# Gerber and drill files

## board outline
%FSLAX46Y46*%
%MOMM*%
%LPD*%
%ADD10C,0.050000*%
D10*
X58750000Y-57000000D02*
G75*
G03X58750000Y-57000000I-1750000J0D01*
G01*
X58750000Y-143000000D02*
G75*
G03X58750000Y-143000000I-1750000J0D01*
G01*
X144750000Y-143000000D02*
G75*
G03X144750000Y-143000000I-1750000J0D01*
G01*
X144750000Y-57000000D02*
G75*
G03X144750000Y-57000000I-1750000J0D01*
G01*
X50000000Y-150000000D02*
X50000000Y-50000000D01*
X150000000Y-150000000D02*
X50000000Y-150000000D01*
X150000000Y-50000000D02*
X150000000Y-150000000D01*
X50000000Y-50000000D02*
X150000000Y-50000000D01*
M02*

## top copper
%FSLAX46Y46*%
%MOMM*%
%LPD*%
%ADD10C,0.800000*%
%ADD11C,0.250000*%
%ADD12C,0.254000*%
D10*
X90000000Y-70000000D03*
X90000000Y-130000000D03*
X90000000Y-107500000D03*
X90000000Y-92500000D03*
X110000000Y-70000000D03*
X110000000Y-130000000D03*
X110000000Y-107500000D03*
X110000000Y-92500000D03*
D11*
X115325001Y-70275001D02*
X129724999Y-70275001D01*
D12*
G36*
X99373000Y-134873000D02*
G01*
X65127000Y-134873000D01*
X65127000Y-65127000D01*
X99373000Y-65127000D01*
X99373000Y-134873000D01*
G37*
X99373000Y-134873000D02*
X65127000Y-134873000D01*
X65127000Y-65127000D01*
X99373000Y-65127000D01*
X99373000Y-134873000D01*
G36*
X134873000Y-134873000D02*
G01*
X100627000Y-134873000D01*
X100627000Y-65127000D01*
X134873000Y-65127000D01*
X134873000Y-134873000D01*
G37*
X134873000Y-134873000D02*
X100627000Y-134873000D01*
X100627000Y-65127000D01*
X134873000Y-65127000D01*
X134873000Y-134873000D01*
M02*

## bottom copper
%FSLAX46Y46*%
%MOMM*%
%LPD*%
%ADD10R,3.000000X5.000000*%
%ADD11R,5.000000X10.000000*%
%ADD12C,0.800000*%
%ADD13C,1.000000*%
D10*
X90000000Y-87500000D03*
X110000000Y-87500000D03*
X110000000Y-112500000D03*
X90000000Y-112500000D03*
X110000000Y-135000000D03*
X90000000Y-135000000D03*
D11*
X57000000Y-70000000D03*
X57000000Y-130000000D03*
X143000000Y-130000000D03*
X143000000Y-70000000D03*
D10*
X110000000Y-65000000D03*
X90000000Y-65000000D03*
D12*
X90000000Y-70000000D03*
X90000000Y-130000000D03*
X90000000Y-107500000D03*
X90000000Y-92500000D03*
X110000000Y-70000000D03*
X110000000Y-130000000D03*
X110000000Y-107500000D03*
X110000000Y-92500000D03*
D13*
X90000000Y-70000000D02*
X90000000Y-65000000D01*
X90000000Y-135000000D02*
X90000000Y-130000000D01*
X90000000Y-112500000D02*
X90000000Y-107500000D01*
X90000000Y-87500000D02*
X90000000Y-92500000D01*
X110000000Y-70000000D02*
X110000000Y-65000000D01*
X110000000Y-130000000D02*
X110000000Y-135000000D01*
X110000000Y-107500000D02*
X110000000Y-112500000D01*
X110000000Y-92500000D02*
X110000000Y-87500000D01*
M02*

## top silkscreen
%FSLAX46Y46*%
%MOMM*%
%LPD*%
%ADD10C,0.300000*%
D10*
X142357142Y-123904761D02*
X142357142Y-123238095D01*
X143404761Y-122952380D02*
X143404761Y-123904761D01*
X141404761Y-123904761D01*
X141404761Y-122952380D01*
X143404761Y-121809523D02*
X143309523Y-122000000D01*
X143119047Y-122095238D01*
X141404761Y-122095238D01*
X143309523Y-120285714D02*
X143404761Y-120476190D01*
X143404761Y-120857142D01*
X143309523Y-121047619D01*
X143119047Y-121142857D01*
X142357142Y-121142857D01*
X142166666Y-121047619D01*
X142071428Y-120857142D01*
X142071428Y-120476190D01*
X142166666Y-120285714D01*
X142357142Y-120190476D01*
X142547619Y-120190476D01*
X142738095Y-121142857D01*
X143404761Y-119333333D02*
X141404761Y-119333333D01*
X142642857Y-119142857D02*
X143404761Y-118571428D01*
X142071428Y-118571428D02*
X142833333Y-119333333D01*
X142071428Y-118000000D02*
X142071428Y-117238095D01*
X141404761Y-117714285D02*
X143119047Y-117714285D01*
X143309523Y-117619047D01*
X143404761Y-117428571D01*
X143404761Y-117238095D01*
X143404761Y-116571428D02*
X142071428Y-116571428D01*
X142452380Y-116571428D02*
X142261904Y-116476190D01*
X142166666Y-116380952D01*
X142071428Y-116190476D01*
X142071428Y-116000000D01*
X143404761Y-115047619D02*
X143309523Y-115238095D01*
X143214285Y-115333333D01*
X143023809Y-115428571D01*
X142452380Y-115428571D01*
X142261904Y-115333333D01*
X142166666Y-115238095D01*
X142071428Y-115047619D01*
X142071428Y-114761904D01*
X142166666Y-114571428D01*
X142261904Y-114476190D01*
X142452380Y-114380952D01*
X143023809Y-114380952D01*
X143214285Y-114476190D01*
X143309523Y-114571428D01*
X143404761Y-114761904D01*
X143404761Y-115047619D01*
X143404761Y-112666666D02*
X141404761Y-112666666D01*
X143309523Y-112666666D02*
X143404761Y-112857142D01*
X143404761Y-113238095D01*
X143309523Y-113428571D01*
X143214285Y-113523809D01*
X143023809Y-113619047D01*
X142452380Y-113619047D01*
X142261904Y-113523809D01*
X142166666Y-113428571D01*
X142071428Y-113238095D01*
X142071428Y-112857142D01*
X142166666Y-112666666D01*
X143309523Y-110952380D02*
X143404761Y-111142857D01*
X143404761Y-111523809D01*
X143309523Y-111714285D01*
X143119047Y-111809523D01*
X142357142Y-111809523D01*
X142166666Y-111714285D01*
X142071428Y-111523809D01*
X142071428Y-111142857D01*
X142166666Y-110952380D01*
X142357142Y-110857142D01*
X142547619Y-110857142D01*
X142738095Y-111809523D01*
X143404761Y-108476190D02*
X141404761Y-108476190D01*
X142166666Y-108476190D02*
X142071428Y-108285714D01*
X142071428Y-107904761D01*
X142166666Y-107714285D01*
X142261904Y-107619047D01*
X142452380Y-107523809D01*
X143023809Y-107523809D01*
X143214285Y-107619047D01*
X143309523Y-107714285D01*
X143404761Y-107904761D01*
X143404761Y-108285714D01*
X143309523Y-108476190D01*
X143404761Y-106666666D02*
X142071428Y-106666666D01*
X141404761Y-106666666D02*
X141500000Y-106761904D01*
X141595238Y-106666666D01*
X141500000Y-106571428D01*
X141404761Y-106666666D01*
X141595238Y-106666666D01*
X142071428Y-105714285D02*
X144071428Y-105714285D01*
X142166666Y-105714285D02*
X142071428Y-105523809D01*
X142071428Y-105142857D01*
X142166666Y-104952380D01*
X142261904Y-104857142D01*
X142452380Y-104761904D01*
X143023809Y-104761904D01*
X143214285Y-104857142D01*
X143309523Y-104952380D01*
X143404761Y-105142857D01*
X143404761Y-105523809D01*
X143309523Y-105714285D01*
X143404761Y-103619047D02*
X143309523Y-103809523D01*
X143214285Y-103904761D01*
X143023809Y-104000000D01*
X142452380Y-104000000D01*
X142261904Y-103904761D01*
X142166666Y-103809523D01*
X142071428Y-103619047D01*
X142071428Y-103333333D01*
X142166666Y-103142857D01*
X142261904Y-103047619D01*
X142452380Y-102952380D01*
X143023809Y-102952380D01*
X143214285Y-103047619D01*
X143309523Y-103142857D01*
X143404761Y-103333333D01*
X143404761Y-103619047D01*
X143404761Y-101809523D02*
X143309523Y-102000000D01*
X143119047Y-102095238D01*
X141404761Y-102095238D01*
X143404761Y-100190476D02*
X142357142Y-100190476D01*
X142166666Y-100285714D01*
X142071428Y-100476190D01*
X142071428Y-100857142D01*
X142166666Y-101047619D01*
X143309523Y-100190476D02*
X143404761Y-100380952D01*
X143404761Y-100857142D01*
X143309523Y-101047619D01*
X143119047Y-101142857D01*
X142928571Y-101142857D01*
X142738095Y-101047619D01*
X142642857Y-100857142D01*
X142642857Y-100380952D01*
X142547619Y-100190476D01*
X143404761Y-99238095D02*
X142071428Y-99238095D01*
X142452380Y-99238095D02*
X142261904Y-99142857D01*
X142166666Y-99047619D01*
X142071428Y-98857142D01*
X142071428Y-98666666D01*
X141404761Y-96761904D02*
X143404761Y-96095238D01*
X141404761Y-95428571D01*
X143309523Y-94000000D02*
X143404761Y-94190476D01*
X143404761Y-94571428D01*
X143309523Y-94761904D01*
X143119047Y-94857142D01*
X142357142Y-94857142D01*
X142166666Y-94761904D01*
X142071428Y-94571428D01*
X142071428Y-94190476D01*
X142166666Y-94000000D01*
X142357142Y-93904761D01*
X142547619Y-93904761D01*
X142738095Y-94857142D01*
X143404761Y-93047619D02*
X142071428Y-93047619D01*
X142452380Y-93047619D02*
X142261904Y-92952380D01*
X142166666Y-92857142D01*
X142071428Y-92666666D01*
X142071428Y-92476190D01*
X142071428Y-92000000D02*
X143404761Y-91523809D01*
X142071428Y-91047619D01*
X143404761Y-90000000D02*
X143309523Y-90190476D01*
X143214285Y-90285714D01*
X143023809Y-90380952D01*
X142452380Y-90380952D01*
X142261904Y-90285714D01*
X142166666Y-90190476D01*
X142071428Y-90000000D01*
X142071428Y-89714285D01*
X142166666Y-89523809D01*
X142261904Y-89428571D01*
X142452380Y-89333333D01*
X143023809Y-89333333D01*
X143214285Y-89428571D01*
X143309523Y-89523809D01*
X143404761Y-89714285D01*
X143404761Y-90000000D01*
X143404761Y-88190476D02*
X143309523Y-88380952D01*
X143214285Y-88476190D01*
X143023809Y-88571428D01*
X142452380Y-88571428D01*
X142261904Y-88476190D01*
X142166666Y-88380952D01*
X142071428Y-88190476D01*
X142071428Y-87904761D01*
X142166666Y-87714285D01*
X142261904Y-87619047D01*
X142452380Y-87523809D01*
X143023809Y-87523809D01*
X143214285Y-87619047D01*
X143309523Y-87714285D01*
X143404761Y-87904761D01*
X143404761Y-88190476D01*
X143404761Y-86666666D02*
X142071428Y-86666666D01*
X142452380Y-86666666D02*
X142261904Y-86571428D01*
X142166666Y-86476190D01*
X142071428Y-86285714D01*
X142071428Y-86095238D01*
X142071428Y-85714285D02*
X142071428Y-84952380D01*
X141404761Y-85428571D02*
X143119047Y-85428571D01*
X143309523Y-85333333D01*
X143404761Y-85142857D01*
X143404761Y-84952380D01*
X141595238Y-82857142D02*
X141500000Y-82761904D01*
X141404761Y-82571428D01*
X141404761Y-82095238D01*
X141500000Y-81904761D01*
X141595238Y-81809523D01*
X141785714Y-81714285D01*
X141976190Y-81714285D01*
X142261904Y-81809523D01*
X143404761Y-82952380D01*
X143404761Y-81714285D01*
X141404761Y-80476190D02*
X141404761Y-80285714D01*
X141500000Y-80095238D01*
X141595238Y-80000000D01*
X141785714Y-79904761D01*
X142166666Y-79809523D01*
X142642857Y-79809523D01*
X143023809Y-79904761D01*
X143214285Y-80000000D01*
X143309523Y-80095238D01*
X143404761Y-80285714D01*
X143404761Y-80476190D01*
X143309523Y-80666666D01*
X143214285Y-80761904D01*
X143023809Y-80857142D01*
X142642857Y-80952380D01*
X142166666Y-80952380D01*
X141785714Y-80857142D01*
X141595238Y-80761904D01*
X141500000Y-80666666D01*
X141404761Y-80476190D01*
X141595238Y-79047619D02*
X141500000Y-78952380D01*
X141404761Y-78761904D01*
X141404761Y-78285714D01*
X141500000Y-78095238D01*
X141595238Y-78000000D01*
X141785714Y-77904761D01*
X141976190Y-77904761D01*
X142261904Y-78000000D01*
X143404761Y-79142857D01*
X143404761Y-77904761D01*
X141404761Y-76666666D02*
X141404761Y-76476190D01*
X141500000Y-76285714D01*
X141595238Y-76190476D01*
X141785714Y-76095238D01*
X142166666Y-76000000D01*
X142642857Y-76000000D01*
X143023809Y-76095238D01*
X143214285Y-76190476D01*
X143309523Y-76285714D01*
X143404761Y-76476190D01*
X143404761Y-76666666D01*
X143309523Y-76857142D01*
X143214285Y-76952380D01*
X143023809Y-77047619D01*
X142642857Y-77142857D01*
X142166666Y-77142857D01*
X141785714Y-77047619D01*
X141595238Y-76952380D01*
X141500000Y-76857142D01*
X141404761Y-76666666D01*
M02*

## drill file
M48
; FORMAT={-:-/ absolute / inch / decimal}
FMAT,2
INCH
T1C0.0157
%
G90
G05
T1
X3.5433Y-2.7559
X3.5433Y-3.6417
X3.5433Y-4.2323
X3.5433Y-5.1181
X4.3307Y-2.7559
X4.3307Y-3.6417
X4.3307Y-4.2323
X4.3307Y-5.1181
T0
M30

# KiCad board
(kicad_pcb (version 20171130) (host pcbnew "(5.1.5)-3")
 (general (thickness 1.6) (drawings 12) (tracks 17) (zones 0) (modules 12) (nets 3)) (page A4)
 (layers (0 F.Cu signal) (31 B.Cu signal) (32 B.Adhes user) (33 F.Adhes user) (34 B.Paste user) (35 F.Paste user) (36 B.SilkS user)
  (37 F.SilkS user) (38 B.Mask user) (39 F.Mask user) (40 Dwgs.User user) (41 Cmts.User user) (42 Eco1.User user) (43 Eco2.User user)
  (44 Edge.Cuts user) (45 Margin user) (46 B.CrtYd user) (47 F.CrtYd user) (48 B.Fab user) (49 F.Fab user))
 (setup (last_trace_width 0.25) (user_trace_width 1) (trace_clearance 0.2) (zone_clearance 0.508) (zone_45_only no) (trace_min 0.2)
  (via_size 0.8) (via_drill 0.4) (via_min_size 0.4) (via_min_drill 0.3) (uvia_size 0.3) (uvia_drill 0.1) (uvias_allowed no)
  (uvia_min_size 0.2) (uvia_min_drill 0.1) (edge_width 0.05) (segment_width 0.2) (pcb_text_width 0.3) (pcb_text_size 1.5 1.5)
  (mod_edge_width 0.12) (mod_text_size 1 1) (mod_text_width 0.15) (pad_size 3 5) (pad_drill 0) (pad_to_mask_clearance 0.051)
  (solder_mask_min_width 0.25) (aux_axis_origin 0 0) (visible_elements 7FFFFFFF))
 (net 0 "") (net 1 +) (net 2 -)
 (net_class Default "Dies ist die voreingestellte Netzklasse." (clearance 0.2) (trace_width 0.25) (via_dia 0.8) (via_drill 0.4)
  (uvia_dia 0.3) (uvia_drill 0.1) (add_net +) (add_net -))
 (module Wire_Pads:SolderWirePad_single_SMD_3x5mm (layer B.Cu) (at 90 87.5)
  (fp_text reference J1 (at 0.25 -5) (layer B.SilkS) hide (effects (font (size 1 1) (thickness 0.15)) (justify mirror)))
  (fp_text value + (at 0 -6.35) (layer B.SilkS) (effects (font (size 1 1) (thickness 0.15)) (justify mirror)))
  (pad 1 smd rect (at 0 0) (size 3 5) (layers B.Cu) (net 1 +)))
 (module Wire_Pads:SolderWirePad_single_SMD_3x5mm (layer B.Cu) (at 110 87.5)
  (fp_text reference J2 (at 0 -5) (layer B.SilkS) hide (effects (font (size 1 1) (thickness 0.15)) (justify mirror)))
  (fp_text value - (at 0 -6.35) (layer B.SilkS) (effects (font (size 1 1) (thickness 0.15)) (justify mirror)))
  (pad 1 smd rect (at 0 0) (size 3 5) (layers B.Cu) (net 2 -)))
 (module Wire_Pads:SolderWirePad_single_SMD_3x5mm (layer B.Cu) (at 110 112.5 180)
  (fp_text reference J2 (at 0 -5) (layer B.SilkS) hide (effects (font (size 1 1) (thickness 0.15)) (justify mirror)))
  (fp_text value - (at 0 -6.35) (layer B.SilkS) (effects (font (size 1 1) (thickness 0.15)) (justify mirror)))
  (pad 1 smd rect (at 0 0 180) (size 3 5) (layers B.Cu) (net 2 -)))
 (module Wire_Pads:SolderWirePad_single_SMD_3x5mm (layer B.Cu) (at 90 112.5 180)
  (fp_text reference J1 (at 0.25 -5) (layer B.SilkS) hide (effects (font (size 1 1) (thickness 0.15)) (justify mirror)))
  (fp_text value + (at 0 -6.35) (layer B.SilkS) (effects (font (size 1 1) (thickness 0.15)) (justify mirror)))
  (pad 1 smd rect (at 0 0 180) (size 3 5) (layers B.Cu) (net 1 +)))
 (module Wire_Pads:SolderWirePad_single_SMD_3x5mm (layer B.Cu) (at 110 135 180)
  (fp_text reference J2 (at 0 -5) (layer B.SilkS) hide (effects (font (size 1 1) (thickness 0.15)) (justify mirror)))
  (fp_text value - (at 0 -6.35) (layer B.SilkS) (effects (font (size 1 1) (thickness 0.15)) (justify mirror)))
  (pad 1 smd rect (at 0 0 180) (size 3 5) (layers B.Cu) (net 2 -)))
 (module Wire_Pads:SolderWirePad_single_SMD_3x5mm (layer B.Cu) (at 90 135 180)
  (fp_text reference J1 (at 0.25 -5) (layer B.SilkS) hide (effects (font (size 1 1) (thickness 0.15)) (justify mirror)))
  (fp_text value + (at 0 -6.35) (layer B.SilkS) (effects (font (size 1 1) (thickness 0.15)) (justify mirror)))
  (pad 1 smd rect (at 0 0 180) (size 3 5) (layers B.Cu) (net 1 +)))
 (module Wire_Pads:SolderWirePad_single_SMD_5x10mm (layer B.Cu) (at 57 70)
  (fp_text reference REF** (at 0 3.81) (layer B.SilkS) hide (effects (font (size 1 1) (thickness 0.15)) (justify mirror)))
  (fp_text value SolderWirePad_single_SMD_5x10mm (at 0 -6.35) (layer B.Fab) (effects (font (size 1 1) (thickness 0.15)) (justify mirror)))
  (pad 1 smd rect (at 0 0) (size 5 10) (layers B.Cu B.Paste B.Mask)))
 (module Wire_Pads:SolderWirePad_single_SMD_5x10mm (layer B.Cu) (at 57 130)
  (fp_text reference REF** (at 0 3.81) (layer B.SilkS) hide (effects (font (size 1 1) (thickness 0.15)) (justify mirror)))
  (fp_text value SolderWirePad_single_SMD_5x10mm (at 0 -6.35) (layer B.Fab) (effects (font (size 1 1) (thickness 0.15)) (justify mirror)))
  (pad 1 smd rect (at 0 0) (size 5 10) (layers B.Cu B.Paste B.Mask)))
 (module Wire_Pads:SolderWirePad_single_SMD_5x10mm (layer B.Cu) (at 143 130)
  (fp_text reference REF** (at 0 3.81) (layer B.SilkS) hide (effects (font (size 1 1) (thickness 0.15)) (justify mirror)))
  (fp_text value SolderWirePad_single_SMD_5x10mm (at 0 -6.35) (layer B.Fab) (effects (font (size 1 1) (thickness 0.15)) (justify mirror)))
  (pad 1 smd rect (at 0 0) (size 5 10) (layers B.Cu B.Paste B.Mask)))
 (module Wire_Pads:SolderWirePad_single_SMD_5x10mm (layer B.Cu) (at 143 70)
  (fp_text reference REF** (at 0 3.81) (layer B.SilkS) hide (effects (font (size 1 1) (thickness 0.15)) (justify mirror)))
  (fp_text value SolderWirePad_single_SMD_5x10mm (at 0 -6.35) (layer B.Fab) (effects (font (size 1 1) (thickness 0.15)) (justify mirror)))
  (pad 1 smd rect (at 0 0) (size 5 10) (layers B.Cu B.Paste B.Mask)))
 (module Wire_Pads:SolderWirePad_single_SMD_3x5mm (layer B.Cu) (at 110 65)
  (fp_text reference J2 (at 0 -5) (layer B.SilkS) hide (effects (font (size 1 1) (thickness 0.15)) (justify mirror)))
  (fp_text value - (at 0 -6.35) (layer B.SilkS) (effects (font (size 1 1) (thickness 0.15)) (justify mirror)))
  (pad 1 smd rect (at 0 0) (size 3 5) (layers B.Cu B.Paste B.Mask) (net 2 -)))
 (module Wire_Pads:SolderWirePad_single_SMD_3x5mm (layer B.Cu) (at 90 65)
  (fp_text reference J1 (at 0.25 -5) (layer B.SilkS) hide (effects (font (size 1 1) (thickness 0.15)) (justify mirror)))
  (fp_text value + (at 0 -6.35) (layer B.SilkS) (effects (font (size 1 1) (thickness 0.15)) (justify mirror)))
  (pad 1 smd rect (at 0 0) (size 3 5) (layers B.Cu B.Paste B.Mask) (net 1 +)))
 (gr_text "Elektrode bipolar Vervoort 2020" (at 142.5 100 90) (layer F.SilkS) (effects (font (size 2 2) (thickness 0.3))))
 (gr_circle (center 57 57) (end 58.75 57) (layer Edge.Cuts) (width 0.05))
 (gr_circle (center 57 143) (end 58.75 143) (layer Edge.Cuts) (width 0.05))
 (gr_circle (center 143 143) (end 144.75 143) (layer Edge.Cuts) (width 0.05))
 (gr_circle (center 143 57) (end 144.75 57) (layer Edge.Cuts) (width 0.05))
 (gr_line (start 50 150) (end 50 50) (layer Edge.Cuts) (width 0.05))
 (gr_line (start 150 150) (end 50 150) (layer Edge.Cuts) (width 0.05))
 (gr_line (start 150 50) (end 150 150) (layer Edge.Cuts) (width 0.05))
 (gr_line (start 50 50) (end 150 50) (layer Edge.Cuts) (width 0.05))
 (via (at 90 70) (size 0.8) (drill 0.4) (layers F.Cu B.Cu) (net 1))
 (segment (start 90 70) (end 90 65) (width 1) (layer B.Cu) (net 1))
 (via (at 90 130) (size 0.8) (drill 0.4) (layers F.Cu B.Cu) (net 1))
 (segment (start 90 135) (end 90 130) (width 1) (layer B.Cu) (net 1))
 (segment (start 90 112.5) (end 90 107.5) (width 1) (layer B.Cu) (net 1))
 (via (at 90 107.5) (size 0.8) (drill 0.4) (layers F.Cu B.Cu) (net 1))
 (segment (start 90 87.5) (end 90 92.5) (width 1) (layer B.Cu) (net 1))
 (via (at 90 92.5) (size 0.8) (drill 0.4) (layers F.Cu B.Cu) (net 1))
 (segment (start 115.325001 70.275001) (end 129.724999 70.275001) (width 0.25) (layer F.Cu) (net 2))
 (via (at 110 70) (size 0.8) (drill 0.4) (layers F.Cu B.Cu) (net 2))
 (via (at 110 130) (size 0.8) (drill 0.4) (layers F.Cu B.Cu) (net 2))
 (segment (start 110 70) (end 110 65) (width 1) (layer B.Cu) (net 2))
 (segment (start 110 130) (end 110 135) (width 1) (layer B.Cu) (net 2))
 (segment (start 110 107.5) (end 110 112.5) (width 1) (layer B.Cu) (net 2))
 (via (at 110 107.5) (size 0.8) (drill 0.4) (layers F.Cu B.Cu) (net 2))
 (segment (start 110 92.5) (end 110 87.5) (width 1) (layer B.Cu) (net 2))
 (via (at 110 92.5) (size 0.8) (drill 0.4) (layers F.Cu B.Cu) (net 2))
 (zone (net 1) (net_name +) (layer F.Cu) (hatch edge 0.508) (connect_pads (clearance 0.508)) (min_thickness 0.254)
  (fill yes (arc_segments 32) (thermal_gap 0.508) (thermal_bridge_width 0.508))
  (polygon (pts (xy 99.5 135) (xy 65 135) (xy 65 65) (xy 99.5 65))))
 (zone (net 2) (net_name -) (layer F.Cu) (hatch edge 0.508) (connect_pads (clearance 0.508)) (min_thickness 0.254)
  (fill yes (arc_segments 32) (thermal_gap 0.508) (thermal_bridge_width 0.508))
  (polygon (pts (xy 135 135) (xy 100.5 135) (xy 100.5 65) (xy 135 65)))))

